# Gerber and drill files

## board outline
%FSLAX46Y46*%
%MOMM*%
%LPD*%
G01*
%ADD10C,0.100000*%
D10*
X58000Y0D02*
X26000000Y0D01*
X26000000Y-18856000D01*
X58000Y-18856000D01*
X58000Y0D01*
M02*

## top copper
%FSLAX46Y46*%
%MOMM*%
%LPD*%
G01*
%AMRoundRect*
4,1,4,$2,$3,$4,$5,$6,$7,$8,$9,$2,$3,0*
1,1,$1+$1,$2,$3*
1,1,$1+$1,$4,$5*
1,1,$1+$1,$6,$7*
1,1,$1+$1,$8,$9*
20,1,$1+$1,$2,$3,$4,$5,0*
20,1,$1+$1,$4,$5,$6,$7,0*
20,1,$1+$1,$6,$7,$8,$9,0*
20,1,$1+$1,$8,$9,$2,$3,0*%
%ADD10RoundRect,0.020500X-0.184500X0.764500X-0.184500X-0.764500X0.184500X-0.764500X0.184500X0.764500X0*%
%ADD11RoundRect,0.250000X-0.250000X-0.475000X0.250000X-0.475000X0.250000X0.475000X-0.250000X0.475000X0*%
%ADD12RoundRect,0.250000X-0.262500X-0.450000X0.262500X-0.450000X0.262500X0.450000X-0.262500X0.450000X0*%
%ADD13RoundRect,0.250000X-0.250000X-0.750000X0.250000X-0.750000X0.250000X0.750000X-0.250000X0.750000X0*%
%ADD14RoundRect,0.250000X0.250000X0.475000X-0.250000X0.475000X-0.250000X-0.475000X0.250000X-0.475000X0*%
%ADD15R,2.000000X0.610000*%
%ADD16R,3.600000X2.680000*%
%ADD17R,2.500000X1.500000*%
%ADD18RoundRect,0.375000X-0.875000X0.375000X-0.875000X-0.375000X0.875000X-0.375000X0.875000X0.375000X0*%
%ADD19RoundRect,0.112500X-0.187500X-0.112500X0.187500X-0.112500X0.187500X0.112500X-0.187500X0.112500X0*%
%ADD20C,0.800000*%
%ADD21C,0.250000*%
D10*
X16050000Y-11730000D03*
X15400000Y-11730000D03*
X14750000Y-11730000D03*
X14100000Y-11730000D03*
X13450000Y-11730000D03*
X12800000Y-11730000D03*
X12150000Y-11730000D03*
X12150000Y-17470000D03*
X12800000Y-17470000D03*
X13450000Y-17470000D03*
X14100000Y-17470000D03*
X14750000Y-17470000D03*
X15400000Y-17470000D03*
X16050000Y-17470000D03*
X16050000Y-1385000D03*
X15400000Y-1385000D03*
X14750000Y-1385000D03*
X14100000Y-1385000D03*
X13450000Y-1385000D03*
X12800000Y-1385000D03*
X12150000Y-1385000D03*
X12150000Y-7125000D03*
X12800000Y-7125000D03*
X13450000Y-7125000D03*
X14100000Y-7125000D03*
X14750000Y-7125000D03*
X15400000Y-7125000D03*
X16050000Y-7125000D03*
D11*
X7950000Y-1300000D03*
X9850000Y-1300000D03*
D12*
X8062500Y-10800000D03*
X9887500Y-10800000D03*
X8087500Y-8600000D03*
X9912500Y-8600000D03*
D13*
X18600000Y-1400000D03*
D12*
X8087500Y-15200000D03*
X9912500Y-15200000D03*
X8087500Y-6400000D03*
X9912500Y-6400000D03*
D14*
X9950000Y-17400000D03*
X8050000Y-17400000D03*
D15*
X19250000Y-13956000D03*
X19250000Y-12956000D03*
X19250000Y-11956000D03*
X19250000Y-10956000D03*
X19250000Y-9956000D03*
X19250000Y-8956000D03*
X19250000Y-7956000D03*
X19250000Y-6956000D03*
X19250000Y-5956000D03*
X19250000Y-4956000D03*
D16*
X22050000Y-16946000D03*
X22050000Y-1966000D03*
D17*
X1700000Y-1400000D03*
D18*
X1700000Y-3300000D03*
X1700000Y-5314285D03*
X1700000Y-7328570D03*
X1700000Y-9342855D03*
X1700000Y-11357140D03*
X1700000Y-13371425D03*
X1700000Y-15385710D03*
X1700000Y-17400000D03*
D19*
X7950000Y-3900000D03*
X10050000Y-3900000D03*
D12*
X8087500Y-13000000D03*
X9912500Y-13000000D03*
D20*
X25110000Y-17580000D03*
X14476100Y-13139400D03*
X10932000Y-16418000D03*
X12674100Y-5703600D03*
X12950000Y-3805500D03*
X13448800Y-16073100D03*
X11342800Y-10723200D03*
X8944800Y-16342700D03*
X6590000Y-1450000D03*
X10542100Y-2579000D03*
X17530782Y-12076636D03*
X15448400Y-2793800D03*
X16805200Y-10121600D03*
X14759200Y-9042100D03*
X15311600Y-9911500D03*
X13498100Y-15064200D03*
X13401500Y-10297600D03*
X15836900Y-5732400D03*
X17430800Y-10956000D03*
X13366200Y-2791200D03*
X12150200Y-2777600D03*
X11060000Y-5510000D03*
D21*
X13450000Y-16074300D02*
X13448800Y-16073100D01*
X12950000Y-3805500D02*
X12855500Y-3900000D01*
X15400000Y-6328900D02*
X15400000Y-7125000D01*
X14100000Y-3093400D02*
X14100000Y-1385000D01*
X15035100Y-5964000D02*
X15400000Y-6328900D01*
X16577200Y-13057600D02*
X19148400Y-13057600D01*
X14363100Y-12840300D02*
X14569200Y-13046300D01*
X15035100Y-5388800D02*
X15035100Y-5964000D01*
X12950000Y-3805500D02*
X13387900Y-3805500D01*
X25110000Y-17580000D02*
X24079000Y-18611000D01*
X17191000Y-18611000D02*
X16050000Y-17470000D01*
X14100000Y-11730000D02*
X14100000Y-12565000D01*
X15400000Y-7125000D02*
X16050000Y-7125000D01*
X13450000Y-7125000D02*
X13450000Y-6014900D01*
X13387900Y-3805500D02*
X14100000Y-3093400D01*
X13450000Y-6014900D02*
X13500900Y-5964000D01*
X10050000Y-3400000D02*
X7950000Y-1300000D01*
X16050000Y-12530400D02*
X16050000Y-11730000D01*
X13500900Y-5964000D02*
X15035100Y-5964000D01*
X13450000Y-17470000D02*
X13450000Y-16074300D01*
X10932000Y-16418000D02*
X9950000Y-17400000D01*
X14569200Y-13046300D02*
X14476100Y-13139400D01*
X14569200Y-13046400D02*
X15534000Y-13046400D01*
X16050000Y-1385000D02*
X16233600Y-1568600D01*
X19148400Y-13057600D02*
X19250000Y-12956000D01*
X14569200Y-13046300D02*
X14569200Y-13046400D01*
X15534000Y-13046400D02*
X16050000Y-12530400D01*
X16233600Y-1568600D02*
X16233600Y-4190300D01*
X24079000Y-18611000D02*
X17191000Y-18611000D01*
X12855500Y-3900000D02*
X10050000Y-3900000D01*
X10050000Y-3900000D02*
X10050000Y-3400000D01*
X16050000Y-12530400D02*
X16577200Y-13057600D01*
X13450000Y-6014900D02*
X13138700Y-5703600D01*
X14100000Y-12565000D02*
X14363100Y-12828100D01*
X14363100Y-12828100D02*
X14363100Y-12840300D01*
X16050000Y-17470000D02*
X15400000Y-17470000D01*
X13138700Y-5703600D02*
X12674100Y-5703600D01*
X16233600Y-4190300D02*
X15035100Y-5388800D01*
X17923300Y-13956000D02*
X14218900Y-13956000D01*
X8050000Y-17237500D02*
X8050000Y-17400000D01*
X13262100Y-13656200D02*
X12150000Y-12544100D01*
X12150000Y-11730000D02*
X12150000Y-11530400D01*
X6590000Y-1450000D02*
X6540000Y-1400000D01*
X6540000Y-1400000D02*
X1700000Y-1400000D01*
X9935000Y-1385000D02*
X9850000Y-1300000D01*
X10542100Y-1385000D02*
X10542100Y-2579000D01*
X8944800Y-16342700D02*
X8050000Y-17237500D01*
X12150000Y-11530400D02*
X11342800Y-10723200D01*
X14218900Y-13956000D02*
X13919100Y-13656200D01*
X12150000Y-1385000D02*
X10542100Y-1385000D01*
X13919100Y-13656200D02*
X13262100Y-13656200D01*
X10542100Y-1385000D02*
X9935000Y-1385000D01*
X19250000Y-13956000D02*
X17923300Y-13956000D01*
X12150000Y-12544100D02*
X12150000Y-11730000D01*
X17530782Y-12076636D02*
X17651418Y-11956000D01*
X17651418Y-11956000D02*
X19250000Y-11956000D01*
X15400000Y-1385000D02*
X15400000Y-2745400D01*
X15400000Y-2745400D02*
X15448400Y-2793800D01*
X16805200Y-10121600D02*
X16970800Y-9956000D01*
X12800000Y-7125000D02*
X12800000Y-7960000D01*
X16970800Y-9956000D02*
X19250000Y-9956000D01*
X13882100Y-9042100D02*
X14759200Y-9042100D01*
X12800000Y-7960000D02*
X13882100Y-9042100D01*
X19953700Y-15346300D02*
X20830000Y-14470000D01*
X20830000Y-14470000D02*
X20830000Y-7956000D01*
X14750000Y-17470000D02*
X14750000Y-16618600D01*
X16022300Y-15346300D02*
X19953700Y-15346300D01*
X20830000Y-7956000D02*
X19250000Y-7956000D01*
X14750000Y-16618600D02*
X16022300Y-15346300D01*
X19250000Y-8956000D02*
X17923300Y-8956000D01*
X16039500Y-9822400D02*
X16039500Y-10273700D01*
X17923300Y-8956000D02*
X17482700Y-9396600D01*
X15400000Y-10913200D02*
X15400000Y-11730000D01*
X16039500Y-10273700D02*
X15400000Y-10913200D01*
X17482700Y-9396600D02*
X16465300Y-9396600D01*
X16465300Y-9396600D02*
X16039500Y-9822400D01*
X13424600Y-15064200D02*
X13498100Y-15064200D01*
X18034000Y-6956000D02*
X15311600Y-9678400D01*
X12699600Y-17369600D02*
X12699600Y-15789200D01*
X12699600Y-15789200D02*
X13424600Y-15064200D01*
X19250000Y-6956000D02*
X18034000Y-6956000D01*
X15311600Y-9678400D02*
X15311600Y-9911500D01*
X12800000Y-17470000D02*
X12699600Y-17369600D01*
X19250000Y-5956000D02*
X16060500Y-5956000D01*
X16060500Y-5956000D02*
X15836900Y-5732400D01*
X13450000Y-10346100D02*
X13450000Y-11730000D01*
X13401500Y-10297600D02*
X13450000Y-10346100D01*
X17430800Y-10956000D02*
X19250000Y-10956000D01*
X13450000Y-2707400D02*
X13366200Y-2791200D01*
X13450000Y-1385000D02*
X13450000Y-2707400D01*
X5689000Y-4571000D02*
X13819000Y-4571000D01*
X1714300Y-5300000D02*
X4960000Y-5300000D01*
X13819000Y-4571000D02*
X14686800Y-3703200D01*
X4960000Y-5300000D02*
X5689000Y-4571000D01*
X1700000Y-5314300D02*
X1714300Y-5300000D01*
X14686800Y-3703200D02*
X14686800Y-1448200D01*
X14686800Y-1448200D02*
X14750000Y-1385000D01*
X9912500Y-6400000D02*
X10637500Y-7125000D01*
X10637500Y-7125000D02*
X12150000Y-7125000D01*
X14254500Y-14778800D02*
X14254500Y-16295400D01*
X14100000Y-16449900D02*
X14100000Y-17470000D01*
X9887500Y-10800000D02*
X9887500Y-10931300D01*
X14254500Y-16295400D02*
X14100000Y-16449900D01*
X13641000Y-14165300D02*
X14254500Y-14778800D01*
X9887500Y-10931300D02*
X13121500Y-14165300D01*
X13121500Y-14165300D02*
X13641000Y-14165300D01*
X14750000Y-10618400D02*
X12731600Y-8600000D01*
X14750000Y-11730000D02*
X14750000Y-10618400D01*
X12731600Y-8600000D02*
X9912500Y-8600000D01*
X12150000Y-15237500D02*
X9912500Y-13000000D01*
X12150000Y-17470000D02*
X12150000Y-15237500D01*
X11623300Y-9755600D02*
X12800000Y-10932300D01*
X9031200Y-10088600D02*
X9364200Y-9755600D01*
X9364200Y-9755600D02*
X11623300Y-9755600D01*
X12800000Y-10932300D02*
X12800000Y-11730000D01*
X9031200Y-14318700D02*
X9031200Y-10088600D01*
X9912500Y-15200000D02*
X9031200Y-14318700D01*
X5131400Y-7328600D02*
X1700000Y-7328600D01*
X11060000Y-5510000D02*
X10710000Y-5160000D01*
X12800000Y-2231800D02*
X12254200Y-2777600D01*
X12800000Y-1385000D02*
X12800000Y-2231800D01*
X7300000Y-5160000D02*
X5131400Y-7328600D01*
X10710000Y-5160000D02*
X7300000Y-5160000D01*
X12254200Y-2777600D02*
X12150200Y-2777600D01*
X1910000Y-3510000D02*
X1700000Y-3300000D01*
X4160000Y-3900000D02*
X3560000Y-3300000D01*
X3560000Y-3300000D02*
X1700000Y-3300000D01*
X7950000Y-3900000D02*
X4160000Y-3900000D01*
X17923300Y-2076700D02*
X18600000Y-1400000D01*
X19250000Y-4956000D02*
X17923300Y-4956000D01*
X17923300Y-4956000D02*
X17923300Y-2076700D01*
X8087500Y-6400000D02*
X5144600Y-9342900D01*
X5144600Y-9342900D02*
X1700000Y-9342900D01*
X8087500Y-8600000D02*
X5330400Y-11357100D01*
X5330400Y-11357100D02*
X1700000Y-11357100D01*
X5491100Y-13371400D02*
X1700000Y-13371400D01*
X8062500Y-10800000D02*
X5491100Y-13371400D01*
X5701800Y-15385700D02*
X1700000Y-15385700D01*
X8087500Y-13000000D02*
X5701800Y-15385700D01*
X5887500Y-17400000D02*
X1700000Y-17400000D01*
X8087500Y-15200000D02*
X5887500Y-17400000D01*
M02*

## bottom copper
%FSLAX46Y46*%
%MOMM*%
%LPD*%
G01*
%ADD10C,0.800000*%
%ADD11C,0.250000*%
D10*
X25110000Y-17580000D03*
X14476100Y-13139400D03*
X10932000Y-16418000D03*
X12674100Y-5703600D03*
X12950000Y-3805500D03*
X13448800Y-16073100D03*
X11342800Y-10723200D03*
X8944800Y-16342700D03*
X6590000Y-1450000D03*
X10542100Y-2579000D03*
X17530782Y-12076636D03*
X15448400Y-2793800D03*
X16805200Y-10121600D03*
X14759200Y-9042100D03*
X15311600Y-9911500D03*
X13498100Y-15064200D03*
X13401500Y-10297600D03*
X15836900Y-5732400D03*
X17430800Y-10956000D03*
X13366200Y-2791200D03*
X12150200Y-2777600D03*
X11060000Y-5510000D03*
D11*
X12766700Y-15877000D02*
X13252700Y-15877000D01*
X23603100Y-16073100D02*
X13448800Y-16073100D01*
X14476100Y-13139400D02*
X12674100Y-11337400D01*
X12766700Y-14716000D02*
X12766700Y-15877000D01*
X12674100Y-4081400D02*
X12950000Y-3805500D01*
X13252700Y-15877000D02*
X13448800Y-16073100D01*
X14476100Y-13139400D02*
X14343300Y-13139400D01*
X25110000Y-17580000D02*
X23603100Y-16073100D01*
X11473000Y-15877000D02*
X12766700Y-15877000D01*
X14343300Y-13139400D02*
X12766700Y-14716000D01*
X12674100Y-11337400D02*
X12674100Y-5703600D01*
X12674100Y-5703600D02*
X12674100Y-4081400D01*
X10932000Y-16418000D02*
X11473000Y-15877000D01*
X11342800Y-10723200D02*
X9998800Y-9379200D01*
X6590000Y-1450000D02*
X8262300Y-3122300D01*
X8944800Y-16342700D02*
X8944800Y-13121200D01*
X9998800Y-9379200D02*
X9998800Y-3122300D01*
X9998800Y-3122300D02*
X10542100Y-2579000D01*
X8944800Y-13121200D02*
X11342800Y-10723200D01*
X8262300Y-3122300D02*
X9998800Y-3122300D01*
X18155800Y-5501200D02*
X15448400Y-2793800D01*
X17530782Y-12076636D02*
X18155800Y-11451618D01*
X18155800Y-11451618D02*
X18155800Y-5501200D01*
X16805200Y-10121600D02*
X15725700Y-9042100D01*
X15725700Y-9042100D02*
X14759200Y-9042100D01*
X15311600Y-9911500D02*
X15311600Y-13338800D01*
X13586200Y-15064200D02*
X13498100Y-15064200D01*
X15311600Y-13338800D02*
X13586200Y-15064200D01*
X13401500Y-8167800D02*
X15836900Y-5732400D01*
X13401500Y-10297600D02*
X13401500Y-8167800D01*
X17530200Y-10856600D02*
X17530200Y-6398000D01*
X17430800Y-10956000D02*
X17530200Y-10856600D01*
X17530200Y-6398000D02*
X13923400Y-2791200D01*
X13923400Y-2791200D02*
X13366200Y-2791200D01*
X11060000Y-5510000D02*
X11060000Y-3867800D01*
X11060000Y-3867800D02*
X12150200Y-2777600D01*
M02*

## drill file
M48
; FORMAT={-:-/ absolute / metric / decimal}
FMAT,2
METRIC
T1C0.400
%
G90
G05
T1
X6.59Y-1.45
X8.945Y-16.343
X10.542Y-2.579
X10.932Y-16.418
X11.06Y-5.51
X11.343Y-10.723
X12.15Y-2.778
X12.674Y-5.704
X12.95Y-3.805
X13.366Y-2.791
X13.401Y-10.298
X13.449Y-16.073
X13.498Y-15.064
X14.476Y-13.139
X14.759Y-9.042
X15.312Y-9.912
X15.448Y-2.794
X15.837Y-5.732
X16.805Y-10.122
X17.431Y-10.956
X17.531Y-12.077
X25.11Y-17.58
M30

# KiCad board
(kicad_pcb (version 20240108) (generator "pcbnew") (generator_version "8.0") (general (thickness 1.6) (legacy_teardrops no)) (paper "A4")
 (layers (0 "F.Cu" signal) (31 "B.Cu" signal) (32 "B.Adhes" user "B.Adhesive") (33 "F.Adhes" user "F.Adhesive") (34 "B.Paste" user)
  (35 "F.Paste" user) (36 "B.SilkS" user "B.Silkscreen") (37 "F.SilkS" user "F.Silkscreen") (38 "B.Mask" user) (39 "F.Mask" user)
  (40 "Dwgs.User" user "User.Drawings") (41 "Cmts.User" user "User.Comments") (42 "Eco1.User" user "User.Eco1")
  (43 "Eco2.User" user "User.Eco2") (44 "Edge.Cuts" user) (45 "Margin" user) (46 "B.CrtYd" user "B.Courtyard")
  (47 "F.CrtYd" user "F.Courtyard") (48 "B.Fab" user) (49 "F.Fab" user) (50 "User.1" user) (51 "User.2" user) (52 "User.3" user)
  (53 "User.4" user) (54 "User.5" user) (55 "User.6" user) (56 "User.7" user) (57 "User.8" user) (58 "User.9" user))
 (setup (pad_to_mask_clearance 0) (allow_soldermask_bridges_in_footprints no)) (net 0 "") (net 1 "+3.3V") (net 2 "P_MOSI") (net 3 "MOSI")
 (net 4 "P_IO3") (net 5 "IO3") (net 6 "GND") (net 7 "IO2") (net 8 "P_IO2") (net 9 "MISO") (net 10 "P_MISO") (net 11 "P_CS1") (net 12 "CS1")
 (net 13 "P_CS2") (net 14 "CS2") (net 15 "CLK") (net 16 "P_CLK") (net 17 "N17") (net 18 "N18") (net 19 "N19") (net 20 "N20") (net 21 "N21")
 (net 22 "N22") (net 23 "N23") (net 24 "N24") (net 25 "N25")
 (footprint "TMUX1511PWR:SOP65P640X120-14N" (layer "F.Cu") (at 14.1 14.6 -90)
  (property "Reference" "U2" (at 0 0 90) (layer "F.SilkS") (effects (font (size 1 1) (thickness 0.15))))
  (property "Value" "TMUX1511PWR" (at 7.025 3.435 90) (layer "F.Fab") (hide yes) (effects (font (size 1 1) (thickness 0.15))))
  (pad "1" smd roundrect (at -2.87 -1.95 270) (size 1.57 0.41) (layers "F.Cu" "F.Paste" "F.Mask") (roundrect_rratio 0.05) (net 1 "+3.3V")
   (solder_mask_margin 0.102))
  (pad "2" smd roundrect (at -2.87 -1.3 270) (size 1.57 0.41) (layers "F.Cu" "F.Paste" "F.Mask") (roundrect_rratio 0.05) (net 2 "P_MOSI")
   (solder_mask_margin 0.102))
  (pad "3" smd roundrect (at -2.87 -0.65 270) (size 1.57 0.41) (layers "F.Cu" "F.Paste" "F.Mask") (roundrect_rratio 0.05) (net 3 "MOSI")
   (solder_mask_margin 0.102))
  (pad "4" smd roundrect (at -2.87 0 270) (size 1.57 0.41) (layers "F.Cu" "F.Paste" "F.Mask") (roundrect_rratio 0.05) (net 1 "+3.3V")
   (solder_mask_margin 0.102))
  (pad "5" smd roundrect (at -2.87 0.65 270) (size 1.57 0.41) (layers "F.Cu" "F.Paste" "F.Mask") (roundrect_rratio 0.05) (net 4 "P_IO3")
   (solder_mask_margin 0.102))
  (pad "6" smd roundrect (at -2.87 1.3 270) (size 1.57 0.41) (layers "F.Cu" "F.Paste" "F.Mask") (roundrect_rratio 0.05) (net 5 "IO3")
   (solder_mask_margin 0.102))
  (pad "7" smd roundrect (at -2.87 1.95 270) (size 1.57 0.41) (layers "F.Cu" "F.Paste" "F.Mask") (roundrect_rratio 0.05) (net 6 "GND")
   (solder_mask_margin 0.102))
  (pad "8" smd roundrect (at 2.87 1.95 270) (size 1.57 0.41) (layers "F.Cu" "F.Paste" "F.Mask") (roundrect_rratio 0.05) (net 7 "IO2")
   (solder_mask_margin 0.102))
  (pad "9" smd roundrect (at 2.87 1.3 270) (size 1.57 0.41) (layers "F.Cu" "F.Paste" "F.Mask") (roundrect_rratio 0.05) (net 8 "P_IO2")
   (solder_mask_margin 0.102))
  (pad "10" smd roundrect (at 2.87 0.65 270) (size 1.57 0.41) (layers "F.Cu" "F.Paste" "F.Mask") (roundrect_rratio 0.05) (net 1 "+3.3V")
   (solder_mask_margin 0.102))
  (pad "11" smd roundrect (at 2.87 0 270) (size 1.57 0.41) (layers "F.Cu" "F.Paste" "F.Mask") (roundrect_rratio 0.05) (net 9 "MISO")
   (solder_mask_margin 0.102))
  (pad "12" smd roundrect (at 2.87 -0.65 270) (size 1.57 0.41) (layers "F.Cu" "F.Paste" "F.Mask") (roundrect_rratio 0.05) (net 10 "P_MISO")
   (solder_mask_margin 0.102))
  (pad "13" smd roundrect (at 2.87 -1.3 270) (size 1.57 0.41) (layers "F.Cu" "F.Paste" "F.Mask") (roundrect_rratio 0.05) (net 1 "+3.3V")
   (solder_mask_margin 0.102))
  (pad "14" smd roundrect (at 2.87 -1.95 270) (size 1.57 0.41) (layers "F.Cu" "F.Paste" "F.Mask") (roundrect_rratio 0.05) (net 1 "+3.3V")
   (solder_mask_margin 0.102)))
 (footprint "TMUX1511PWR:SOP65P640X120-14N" (layer "F.Cu") (at 14.1 4.255 -90)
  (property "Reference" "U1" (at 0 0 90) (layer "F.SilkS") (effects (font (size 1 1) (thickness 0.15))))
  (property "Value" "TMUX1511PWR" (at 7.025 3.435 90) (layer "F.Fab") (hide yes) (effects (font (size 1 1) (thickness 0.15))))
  (pad "1" smd roundrect (at -2.87 -1.95 270) (size 1.57 0.41) (layers "F.Cu" "F.Paste" "F.Mask") (roundrect_rratio 0.05) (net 1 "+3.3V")
   (solder_mask_margin 0.102))
  (pad "2" smd roundrect (at -2.87 -1.3 270) (size 1.57 0.41) (layers "F.Cu" "F.Paste" "F.Mask") (roundrect_rratio 0.05) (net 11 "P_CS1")
   (solder_mask_margin 0.102))
  (pad "3" smd roundrect (at -2.87 -0.65 270) (size 1.57 0.41) (layers "F.Cu" "F.Paste" "F.Mask") (roundrect_rratio 0.05) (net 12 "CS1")
   (solder_mask_margin 0.102))
  (pad "4" smd roundrect (at -2.87 0 270) (size 1.57 0.41) (layers "F.Cu" "F.Paste" "F.Mask") (roundrect_rratio 0.05) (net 1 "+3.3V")
   (solder_mask_margin 0.102))
  (pad "5" smd roundrect (at -2.87 0.65 270) (size 1.57 0.41) (layers "F.Cu" "F.Paste" "F.Mask") (roundrect_rratio 0.05) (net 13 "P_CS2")
   (solder_mask_margin 0.102))
  (pad "6" smd roundrect (at -2.87 1.3 270) (size 1.57 0.41) (layers "F.Cu" "F.Paste" "F.Mask") (roundrect_rratio 0.05) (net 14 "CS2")
   (solder_mask_margin 0.102))
  (pad "7" smd roundrect (at -2.87 1.95 270) (size 1.57 0.41) (layers "F.Cu" "F.Paste" "F.Mask") (roundrect_rratio 0.05) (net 6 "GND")
   (solder_mask_margin 0.102))
  (pad "8" smd roundrect (at 2.87 1.95 270) (size 1.57 0.41) (layers "F.Cu" "F.Paste" "F.Mask") (roundrect_rratio 0.05) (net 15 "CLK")
   (solder_mask_margin 0.102))
  (pad "9" smd roundrect (at 2.87 1.3 270) (size 1.57 0.41) (layers "F.Cu" "F.Paste" "F.Mask") (roundrect_rratio 0.05) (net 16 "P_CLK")
   (solder_mask_margin 0.102))
  (pad "10" smd roundrect (at 2.87 0.65 270) (size 1.57 0.41) (layers "F.Cu" "F.Paste" "F.Mask") (roundrect_rratio 0.05) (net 1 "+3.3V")
   (solder_mask_margin 0.102))
  (pad "11" smd roundrect (at 2.87 0 270) (size 1.57 0.41) (layers "F.Cu" "F.Paste" "F.Mask") (roundrect_rratio 0.05) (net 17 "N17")
   (solder_mask_margin 0.102))
  (pad "12" smd roundrect (at 2.87 -0.65 270) (size 1.57 0.41) (layers "F.Cu" "F.Paste" "F.Mask") (roundrect_rratio 0.05) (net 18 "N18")
   (solder_mask_margin 0.102))
  (pad "13" smd roundrect (at 2.87 -1.3 270) (size 1.57 0.41) (layers "F.Cu" "F.Paste" "F.Mask") (roundrect_rratio 0.05) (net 1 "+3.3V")
   (solder_mask_margin 0.102))
  (pad "14" smd roundrect (at 2.87 -1.95 270) (size 1.57 0.41) (layers "F.Cu" "F.Paste" "F.Mask") (roundrect_rratio 0.05) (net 1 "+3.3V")
   (solder_mask_margin 0.102)))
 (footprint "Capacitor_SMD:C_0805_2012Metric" (layer "F.Cu") (at 8.9 1.3)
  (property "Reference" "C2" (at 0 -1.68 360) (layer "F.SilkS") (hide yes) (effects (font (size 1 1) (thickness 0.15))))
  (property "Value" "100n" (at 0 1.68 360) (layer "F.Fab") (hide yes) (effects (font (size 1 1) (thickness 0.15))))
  (pad "1" smd roundrect (at -0.95 0) (size 1 1.45) (layers "F.Cu" "F.Paste" "F.Mask") (roundrect_rratio 0.25) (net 1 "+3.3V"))
  (pad "2" smd roundrect (at 0.95 0) (size 1 1.45) (layers "F.Cu" "F.Paste" "F.Mask") (roundrect_rratio 0.25) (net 6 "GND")))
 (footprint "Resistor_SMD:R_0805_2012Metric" (layer "F.Cu") (at 8.975 10.8)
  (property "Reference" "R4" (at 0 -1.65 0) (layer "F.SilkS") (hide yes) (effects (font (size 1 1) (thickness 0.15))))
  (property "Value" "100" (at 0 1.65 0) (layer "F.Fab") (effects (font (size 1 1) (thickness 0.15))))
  (pad "1" smd roundrect (at -0.9125 0) (size 1.025 1.4) (layers "F.Cu" "F.Paste" "F.Mask") (roundrect_rratio 0.243902439) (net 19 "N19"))
  (pad "2" smd roundrect (at 0.9125 0) (size 1.025 1.4) (layers "F.Cu" "F.Paste" "F.Mask") (roundrect_rratio 0.243902439) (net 9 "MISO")))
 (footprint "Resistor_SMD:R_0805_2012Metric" (layer "F.Cu") (at 9 8.6)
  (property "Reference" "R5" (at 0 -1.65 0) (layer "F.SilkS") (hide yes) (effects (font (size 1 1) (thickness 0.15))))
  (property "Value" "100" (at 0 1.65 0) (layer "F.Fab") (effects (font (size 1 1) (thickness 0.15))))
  (pad "1" smd roundrect (at -0.9125 0) (size 1.025 1.4) (layers "F.Cu" "F.Paste" "F.Mask") (roundrect_rratio 0.243902439) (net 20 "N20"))
  (pad "2" smd roundrect (at 0.9125 0) (size 1.025 1.4) (layers "F.Cu" "F.Paste" "F.Mask") (roundrect_rratio 0.243902439) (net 3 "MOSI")))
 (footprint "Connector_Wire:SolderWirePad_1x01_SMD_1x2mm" (layer "F.Cu") (at 18.6 1.4)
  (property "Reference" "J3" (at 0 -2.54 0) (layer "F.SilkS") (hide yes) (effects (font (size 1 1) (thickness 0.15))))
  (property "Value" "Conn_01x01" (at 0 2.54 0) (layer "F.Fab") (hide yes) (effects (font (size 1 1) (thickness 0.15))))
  (pad "1" smd roundrect (at 0 0) (size 1 2) (layers "F.Cu" "F.Paste" "F.Mask") (roundrect_rratio 0.25) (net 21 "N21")))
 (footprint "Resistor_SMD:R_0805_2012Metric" (layer "F.Cu") (at 9 15.2)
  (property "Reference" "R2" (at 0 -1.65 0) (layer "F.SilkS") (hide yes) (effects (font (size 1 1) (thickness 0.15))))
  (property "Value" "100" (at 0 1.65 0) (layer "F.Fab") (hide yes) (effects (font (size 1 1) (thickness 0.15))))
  (pad "1" smd roundrect (at -0.9125 0) (size 1.025 1.4) (layers "F.Cu" "F.Paste" "F.Mask") (roundrect_rratio 0.243902439) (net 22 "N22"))
  (pad "2" smd roundrect (at 0.9125 0) (size 1.025 1.4) (layers "F.Cu" "F.Paste" "F.Mask") (roundrect_rratio 0.243902439) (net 5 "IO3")))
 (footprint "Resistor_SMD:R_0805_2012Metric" (layer "F.Cu") (at 9 6.4)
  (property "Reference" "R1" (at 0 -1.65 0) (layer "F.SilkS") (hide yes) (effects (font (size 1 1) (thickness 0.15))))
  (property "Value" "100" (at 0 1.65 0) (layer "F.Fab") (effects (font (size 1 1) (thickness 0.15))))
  (pad "1" smd roundrect (at -0.9125 0) (size 1.025 1.4) (layers "F.Cu" "F.Paste" "F.Mask") (roundrect_rratio 0.243902439) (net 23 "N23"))
  (pad "2" smd roundrect (at 0.9125 0) (size 1.025 1.4) (layers "F.Cu" "F.Paste" "F.Mask") (roundrect_rratio 0.243902439) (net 15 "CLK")))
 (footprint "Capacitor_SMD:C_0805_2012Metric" (layer "F.Cu") (at 9 17.4 180)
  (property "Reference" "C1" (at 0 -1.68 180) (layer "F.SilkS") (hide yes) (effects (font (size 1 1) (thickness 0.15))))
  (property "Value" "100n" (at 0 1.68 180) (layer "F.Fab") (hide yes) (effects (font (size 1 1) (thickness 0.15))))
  (pad "1" smd roundrect (at -0.95 0 180) (size 1 1.45) (layers "F.Cu" "F.Paste" "F.Mask") (roundrect_rratio 0.25) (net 1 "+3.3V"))
  (pad "2" smd roundrect (at 0.95 0 180) (size 1 1.45) (layers "F.Cu" "F.Paste" "F.Mask") (roundrect_rratio 0.25) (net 6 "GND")))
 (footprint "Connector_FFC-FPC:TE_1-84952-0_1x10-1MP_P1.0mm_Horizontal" (layer "F.Cu") (at 21.05 9.456 90)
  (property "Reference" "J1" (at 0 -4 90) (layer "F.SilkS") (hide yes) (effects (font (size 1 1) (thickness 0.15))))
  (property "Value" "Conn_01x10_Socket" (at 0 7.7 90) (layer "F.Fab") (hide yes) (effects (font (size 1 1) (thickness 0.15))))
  (pad "1" smd rect (at -4.5 -1.8 90) (size 0.61 2) (layers "F.Cu" "F.Paste" "F.Mask") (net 6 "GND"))
  (pad "2" smd rect (at -3.5 -1.8 90) (size 0.61 2) (layers "F.Cu" "F.Paste" "F.Mask") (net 1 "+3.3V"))
  (pad "3" smd rect (at -2.5 -1.8 90) (size 0.61 2) (layers "F.Cu" "F.Paste" "F.Mask") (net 11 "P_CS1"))
  (pad "4" smd rect (at -1.5 -1.8 90) (size 0.61 2) (layers "F.Cu" "F.Paste" "F.Mask") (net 13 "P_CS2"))
  (pad "5" smd rect (at -0.5 -1.8 90) (size 0.61 2) (layers "F.Cu" "F.Paste" "F.Mask") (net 16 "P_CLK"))
  (pad "6" smd rect (at 0.5 -1.8 90) (size 0.61 2) (layers "F.Cu" "F.Paste" "F.Mask") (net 2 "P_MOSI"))
  (pad "7" smd rect (at 1.5 -1.8 90) (size 0.61 2) (layers "F.Cu" "F.Paste" "F.Mask") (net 10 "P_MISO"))
  (pad "8" smd rect (at 2.5 -1.8 90) (size 0.61 2) (layers "F.Cu" "F.Paste" "F.Mask") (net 8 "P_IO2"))
  (pad "9" smd rect (at 3.5 -1.8 90) (size 0.61 2) (layers "F.Cu" "F.Paste" "F.Mask") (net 4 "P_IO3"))
  (pad "10" smd rect (at 4.5 -1.8 90) (size 0.61 2) (layers "F.Cu" "F.Paste" "F.Mask") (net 21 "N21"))
  (pad "MP" smd rect (at -7.49 1 90) (size 2.68 3.6) (layers "F.Cu" "F.Paste" "F.Mask"))
  (pad "MP" smd rect (at 7.49 1 90) (size 2.68 3.6) (layers "F.Cu" "F.Paste" "F.Mask")))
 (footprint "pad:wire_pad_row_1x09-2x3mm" (layer "F.Cu") (at 1.7 1.4 -90)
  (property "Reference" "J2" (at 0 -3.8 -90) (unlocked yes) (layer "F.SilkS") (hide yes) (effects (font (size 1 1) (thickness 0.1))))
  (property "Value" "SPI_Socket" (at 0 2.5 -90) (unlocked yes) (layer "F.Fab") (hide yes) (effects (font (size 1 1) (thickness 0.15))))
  (pad "1" smd rect (at 0 0 270) (size 1.5 2.5) (layers "F.Cu" "F.Paste" "F.Mask") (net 6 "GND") (thermal_bridge_angle 45))
  (pad "2" smd roundrect (at 1.9 0 270) (size 1.5 2.5) (layers "F.Cu" "F.Paste" "F.Mask") (roundrect_rratio 0.25) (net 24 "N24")
   (thermal_bridge_angle 45))
  (pad "3" smd roundrect (at 3.914285 0 270) (size 1.5 2.5) (layers "F.Cu" "F.Paste" "F.Mask") (roundrect_rratio 0.25) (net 12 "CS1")
   (thermal_bridge_angle 45))
  (pad "4" smd roundrect (at 5.92857 0 270) (size 1.5 2.5) (layers "F.Cu" "F.Paste" "F.Mask") (roundrect_rratio 0.25) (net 14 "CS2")
   (thermal_bridge_angle 45))
  (pad "5" smd roundrect (at 7.942855 0 270) (size 1.5 2.5) (layers "F.Cu" "F.Paste" "F.Mask") (roundrect_rratio 0.25) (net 23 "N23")
   (thermal_bridge_angle 45))
  (pad "6" smd roundrect (at 9.95714 0 270) (size 1.5 2.5) (layers "F.Cu" "F.Paste" "F.Mask") (roundrect_rratio 0.25) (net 20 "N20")
   (thermal_bridge_angle 45))
  (pad "7" smd roundrect (at 11.971425 0 270) (size 1.5 2.5) (layers "F.Cu" "F.Paste" "F.Mask") (roundrect_rratio 0.25) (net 19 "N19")
   (thermal_bridge_angle 45))
  (pad "8" smd roundrect (at 13.98571 0 270) (size 1.5 2.5) (layers "F.Cu" "F.Paste" "F.Mask") (roundrect_rratio 0.25) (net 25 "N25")
   (thermal_bridge_angle 45))
  (pad "9" smd roundrect (at 16 0 270) (size 1.5 2.5) (layers "F.Cu" "F.Paste" "F.Mask") (roundrect_rratio 0.25) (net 22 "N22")
   (thermal_bridge_angle 45)))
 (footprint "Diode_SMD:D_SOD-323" (layer "F.Cu") (at 9 3.9)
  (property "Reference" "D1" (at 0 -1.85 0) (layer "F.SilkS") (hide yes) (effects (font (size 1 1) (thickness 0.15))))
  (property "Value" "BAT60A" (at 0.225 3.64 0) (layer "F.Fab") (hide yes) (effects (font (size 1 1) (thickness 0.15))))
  (pad "1" smd roundrect (at -1.05 0) (size 0.6 0.45) (layers "F.Cu" "F.Paste" "F.Mask") (roundrect_rratio 0.25) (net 24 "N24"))
  (pad "2" smd roundrect (at 1.05 0) (size 0.6 0.45) (layers "F.Cu" "F.Paste" "F.Mask") (roundrect_rratio 0.25) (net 1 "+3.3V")))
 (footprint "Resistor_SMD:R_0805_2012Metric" (layer "F.Cu") (at 9 13)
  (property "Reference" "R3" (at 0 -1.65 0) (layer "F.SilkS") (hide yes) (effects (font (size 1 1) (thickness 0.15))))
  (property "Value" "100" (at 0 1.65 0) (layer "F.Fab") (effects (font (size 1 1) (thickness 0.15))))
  (pad "1" smd roundrect (at -0.9125 0) (size 1.025 1.4) (layers "F.Cu" "F.Paste" "F.Mask") (roundrect_rratio 0.243902439) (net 25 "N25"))
  (pad "2" smd roundrect (at 0.9125 0) (size 1.025 1.4) (layers "F.Cu" "F.Paste" "F.Mask") (roundrect_rratio 0.243902439) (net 7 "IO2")))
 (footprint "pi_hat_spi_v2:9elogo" (layer "B.Cu") (at 21 14.9 180)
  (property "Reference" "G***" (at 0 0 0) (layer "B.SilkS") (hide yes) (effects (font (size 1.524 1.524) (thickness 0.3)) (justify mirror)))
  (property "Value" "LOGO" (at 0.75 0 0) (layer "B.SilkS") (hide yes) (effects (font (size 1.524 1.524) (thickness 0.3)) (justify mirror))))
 (gr_rect (start 0.058 0) (end 26 18.856) (stroke (width 0.1) (type default)) (fill none) (layer "Edge.Cuts"))
 (segment (start 13.45 16.0743) (end 13.4488 16.0731) (width 0.25) (layer "F.Cu") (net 1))
 (segment (start 12.95 3.8055) (end 12.8555 3.9) (width 0.25) (layer "F.Cu") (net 1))
 (segment (start 15.4 6.3289) (end 15.4 7.125) (width 0.25) (layer "F.Cu") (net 1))
 (segment (start 14.1 3.0934) (end 14.1 1.385) (width 0.25) (layer "F.Cu") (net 1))
 (segment (start 15.0351 5.964) (end 15.4 6.3289) (width 0.25) (layer "F.Cu") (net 1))
 (segment (start 16.5772 13.0576) (end 19.1484 13.0576) (width 0.25) (layer "F.Cu") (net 1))
 (segment (start 14.3631 12.8403) (end 14.5692 13.0463) (width 0.25) (layer "F.Cu") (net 1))
 (segment (start 15.0351 5.3888) (end 15.0351 5.964) (width 0.25) (layer "F.Cu") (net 1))
 (segment (start 12.95 3.8055) (end 13.3879 3.8055) (width 0.25) (layer "F.Cu") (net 1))
 (segment (start 25.11 17.58) (end 24.079 18.611) (width 0.25) (layer "F.Cu") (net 1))
 (segment (start 17.191 18.611) (end 16.05 17.47) (width 0.25) (layer "F.Cu") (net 1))
 (segment (start 14.1 11.73) (end 14.1 12.565) (width 0.25) (layer "F.Cu") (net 1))
 (segment (start 15.4 7.125) (end 16.05 7.125) (width 0.25) (layer "F.Cu") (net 1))
 (segment (start 13.45 7.125) (end 13.45 6.0149) (width 0.25) (layer "F.Cu") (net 1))
 (segment (start 13.3879 3.8055) (end 14.1 3.0934) (width 0.25) (layer "F.Cu") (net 1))
 (segment (start 13.45 6.0149) (end 13.5009 5.964) (width 0.25) (layer "F.Cu") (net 1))
 (segment (start 10.05 3.4) (end 7.95 1.3) (width 0.25) (layer "F.Cu") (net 1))
 (segment (start 16.05 12.5304) (end 16.05 11.73) (width 0.25) (layer "F.Cu") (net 1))
 (segment (start 13.5009 5.964) (end 15.0351 5.964) (width 0.25) (layer "F.Cu") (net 1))
 (segment (start 13.45 17.47) (end 13.45 16.0743) (width 0.25) (layer "F.Cu") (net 1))
 (segment (start 10.932 16.418) (end 9.95 17.4) (width 0.25) (layer "F.Cu") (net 1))
 (segment (start 14.5692 13.0463) (end 14.4761 13.1394) (width 0.25) (layer "F.Cu") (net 1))
 (segment (start 14.5692 13.0464) (end 15.534 13.0464) (width 0.25) (layer "F.Cu") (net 1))
 (segment (start 16.05 1.385) (end 16.2336 1.5686) (width 0.25) (layer "F.Cu") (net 1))
 (segment (start 19.1484 13.0576) (end 19.25 12.956) (width 0.25) (layer "F.Cu") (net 1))
 (segment (start 14.5692 13.0463) (end 14.5692 13.0464) (width 0.25) (layer "F.Cu") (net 1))
 (segment (start 15.534 13.0464) (end 16.05 12.5304) (width 0.25) (layer "F.Cu") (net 1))
 (segment (start 16.2336 1.5686) (end 16.2336 4.1903) (width 0.25) (layer "F.Cu") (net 1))
 (segment (start 24.079 18.611) (end 17.191 18.611) (width 0.25) (layer "F.Cu") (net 1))
 (segment (start 12.8555 3.9) (end 10.05 3.9) (width 0.25) (layer "F.Cu") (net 1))
 (segment (start 10.05 3.9) (end 10.05 3.4) (width 0.25) (layer "F.Cu") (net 1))
 (segment (start 16.05 12.5304) (end 16.5772 13.0576) (width 0.25) (layer "F.Cu") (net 1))
 (segment (start 13.45 6.0149) (end 13.1387 5.7036) (width 0.25) (layer "F.Cu") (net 1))
 (segment (start 14.1 12.565) (end 14.3631 12.8281) (width 0.25) (layer "F.Cu") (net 1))
 (segment (start 14.3631 12.8281) (end 14.3631 12.8403) (width 0.25) (layer "F.Cu") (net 1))
 (segment (start 16.05 17.47) (end 15.4 17.47) (width 0.25) (layer "F.Cu") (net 1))
 (segment (start 13.1387 5.7036) (end 12.6741 5.7036) (width 0.25) (layer "F.Cu") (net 1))
 (segment (start 16.2336 4.1903) (end 15.0351 5.3888) (width 0.25) (layer "F.Cu") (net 1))
 (via (at 25.11 17.58) (size 0.8) (drill 0.4) (layers "F.Cu" "B.Cu") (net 1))
 (via (at 14.4761 13.1394) (size 0.8) (drill 0.4) (layers "F.Cu" "B.Cu") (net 1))
 (via (at 10.932 16.418) (size 0.8) (drill 0.4) (layers "F.Cu" "B.Cu") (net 1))
 (via (at 12.6741 5.7036) (size 0.8) (drill 0.4) (layers "F.Cu" "B.Cu") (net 1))
 (via (at 12.95 3.8055) (size 0.8) (drill 0.4) (layers "F.Cu" "B.Cu") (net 1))
 (via (at 13.4488 16.0731) (size 0.8) (drill 0.4) (layers "F.Cu" "B.Cu") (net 1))
 (segment (start 12.7667 15.877) (end 13.2527 15.877) (width 0.25) (layer "B.Cu") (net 1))
 (segment (start 23.6031 16.0731) (end 13.4488 16.0731) (width 0.25) (layer "B.Cu") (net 1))
 (segment (start 14.4761 13.1394) (end 12.6741 11.3374) (width 0.25) (layer "B.Cu") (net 1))
 (segment (start 12.7667 14.716) (end 12.7667 15.877) (width 0.25) (layer "B.Cu") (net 1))
 (segment (start 12.6741 4.0814) (end 12.95 3.8055) (width 0.25) (layer "B.Cu") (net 1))
 (segment (start 13.2527 15.877) (end 13.4488 16.0731) (width 0.25) (layer "B.Cu") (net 1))
 (segment (start 14.4761 13.1394) (end 14.3433 13.1394) (width 0.25) (layer "B.Cu") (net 1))
 (segment (start 25.11 17.58) (end 23.6031 16.0731) (width 0.25) (layer "B.Cu") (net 1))
 (segment (start 11.473 15.877) (end 12.7667 15.877) (width 0.25) (layer "B.Cu") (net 1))
 (segment (start 14.3433 13.1394) (end 12.7667 14.716) (width 0.25) (layer "B.Cu") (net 1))
 (segment (start 12.6741 11.3374) (end 12.6741 5.7036) (width 0.25) (layer "B.Cu") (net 1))
 (segment (start 12.6741 5.7036) (end 12.6741 4.0814) (width 0.25) (layer "B.Cu") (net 1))
 (segment (start 10.932 16.418) (end 11.473 15.877) (width 0.25) (layer "B.Cu") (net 1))
 (segment (start 17.9233 13.956) (end 14.2189 13.956) (width 0.25) (layer "F.Cu") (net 6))
 (segment (start 8.05 17.2375) (end 8.05 17.4) (width 0.25) (layer "F.Cu") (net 6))
 (segment (start 13.2621 13.6562) (end 12.15 12.5441) (width 0.25) (layer "F.Cu") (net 6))
 (segment (start 12.15 11.73) (end 12.15 11.5304) (width 0.25) (layer "F.Cu") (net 6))
 (segment (start 6.59 1.45) (end 6.54 1.4) (width 0.25) (layer "F.Cu") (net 6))
 (segment (start 6.54 1.4) (end 1.7 1.4) (width 0.25) (layer "F.Cu") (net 6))
 (segment (start 9.935 1.385) (end 9.85 1.3) (width 0.25) (layer "F.Cu") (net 6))
 (segment (start 10.5421 1.385) (end 10.5421 2.579) (width 0.25) (layer "F.Cu") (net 6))
 (segment (start 8.9448 16.3427) (end 8.05 17.2375) (width 0.25) (layer "F.Cu") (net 6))
 (segment (start 12.15 11.5304) (end 11.3428 10.7232) (width 0.25) (layer "F.Cu") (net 6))
 (segment (start 14.2189 13.956) (end 13.9191 13.6562) (width 0.25) (layer "F.Cu") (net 6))
 (segment (start 12.15 1.385) (end 10.5421 1.385) (width 0.25) (layer "F.Cu") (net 6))
 (segment (start 13.9191 13.6562) (end 13.2621 13.6562) (width 0.25) (layer "F.Cu") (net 6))
 (segment (start 10.5421 1.385) (end 9.935 1.385) (width 0.25) (layer "F.Cu") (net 6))
 (segment (start 19.25 13.956) (end 17.9233 13.956) (width 0.25) (layer "F.Cu") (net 6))
 (segment (start 12.15 12.5441) (end 12.15 11.73) (width 0.25) (layer "F.Cu") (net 6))
 (via (at 11.3428 10.7232) (size 0.8) (drill 0.4) (layers "F.Cu" "B.Cu") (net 6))
 (via (at 8.9448 16.3427) (size 0.8) (drill 0.4) (layers "F.Cu" "B.Cu") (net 6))
 (via (at 6.59 1.45) (size 0.8) (drill 0.4) (layers "F.Cu" "B.Cu") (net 6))
 (via (at 10.5421 2.579) (size 0.8) (drill 0.4) (layers "F.Cu" "B.Cu") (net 6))
 (segment (start 11.3428 10.7232) (end 9.9988 9.3792) (width 0.25) (layer "B.Cu") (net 6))
 (segment (start 6.59 1.45) (end 8.2623 3.1223) (width 0.25) (layer "B.Cu") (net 6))
 (segment (start 8.9448 16.3427) (end 8.9448 13.1212) (width 0.25) (layer "B.Cu") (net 6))
 (segment (start 9.9988 9.3792) (end 9.9988 3.1223) (width 0.25) (layer "B.Cu") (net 6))
 (segment (start 9.9988 3.1223) (end 10.5421 2.579) (width 0.25) (layer "B.Cu") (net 6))
 (segment (start 8.9448 13.1212) (end 11.3428 10.7232) (width 0.25) (layer "B.Cu") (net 6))
 (segment (start 8.2623 3.1223) (end 9.9988 3.1223) (width 0.25) (layer "B.Cu") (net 6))
 (segment (start 17.530782 12.076636) (end 17.651418 11.956) (width 0.25) (layer "F.Cu") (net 11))
 (segment (start 17.651418 11.956) (end 19.25 11.956) (width 0.25) (layer "F.Cu") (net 11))
 (segment (start 15.4 1.385) (end 15.4 2.7454) (width 0.25) (layer "F.Cu") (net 11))
 (segment (start 15.4 2.7454) (end 15.4484 2.7938) (width 0.25) (layer "F.Cu") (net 11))
 (via (at 17.530782 12.076636) (size 0.8) (drill 0.4) (layers "F.Cu" "B.Cu") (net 11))
 (via (at 15.4484 2.7938) (size 0.8) (drill 0.4) (layers "F.Cu" "B.Cu") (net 11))
 (segment (start 18.1558 5.5012) (end 15.4484 2.7938) (width 0.25) (layer "B.Cu") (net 11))
 (segment (start 17.530782 12.076636) (end 18.1558 11.451618) (width 0.25) (layer "B.Cu") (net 11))
 (segment (start 18.1558 11.451618) (end 18.1558 5.5012) (width 0.25) (layer "B.Cu") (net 11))
 (segment (start 16.8052 10.1216) (end 16.9708 9.956) (width 0.25) (layer "F.Cu") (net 16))
 (segment (start 12.8 7.125) (end 12.8 7.96) (width 0.25) (layer "F.Cu") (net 16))
 (segment (start 16.9708 9.956) (end 19.25 9.956) (width 0.25) (layer "F.Cu") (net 16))
 (segment (start 13.8821 9.0421) (end 14.7592 9.0421) (width 0.25) (layer "F.Cu") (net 16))
 (segment (start 12.8 7.96) (end 13.8821 9.0421) (width 0.25) (layer "F.Cu") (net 16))
 (via (at 16.8052 10.1216) (size 0.8) (drill 0.4) (layers "F.Cu" "B.Cu") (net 16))
 (via (at 14.7592 9.0421) (size 0.8) (drill 0.4) (layers "F.Cu" "B.Cu") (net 16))
 (segment (start 16.8052 10.1216) (end 15.7257 9.0421) (width 0.25) (layer "B.Cu") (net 16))
 (segment (start 15.7257 9.0421) (end 14.7592 9.0421) (width 0.25) (layer "B.Cu") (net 16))
 (segment (start 19.9537 15.3463) (end 20.83 14.47) (width 0.25) (layer "F.Cu") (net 10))
 (segment (start 20.83 14.47) (end 20.83 7.956) (width 0.25) (layer "F.Cu") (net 10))
 (segment (start 14.75 17.47) (end 14.75 16.6186) (width 0.25) (layer "F.Cu") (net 10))
 (segment (start 16.0223 15.3463) (end 19.9537 15.3463) (width 0.25) (layer "F.Cu") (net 10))
 (segment (start 20.83 7.956) (end 19.25 7.956) (width 0.25) (layer "F.Cu") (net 10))
 (segment (start 14.75 16.6186) (end 16.0223 15.3463) (width 0.25) (layer "F.Cu") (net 10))
 (segment (start 19.25 8.956) (end 17.9233 8.956) (width 0.25) (layer "F.Cu") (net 2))
 (segment (start 16.0395 9.8224) (end 16.0395 10.2737) (width 0.25) (layer "F.Cu") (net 2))
 (segment (start 17.9233 8.956) (end 17.4827 9.3966) (width 0.25) (layer "F.Cu") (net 2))
 (segment (start 15.4 10.9132) (end 15.4 11.73) (width 0.25) (layer "F.Cu") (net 2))
 (segment (start 16.0395 10.2737) (end 15.4 10.9132) (width 0.25) (layer "F.Cu") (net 2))
 (segment (start 17.4827 9.3966) (end 16.4653 9.3966) (width 0.25) (layer "F.Cu") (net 2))
 (segment (start 16.4653 9.3966) (end 16.0395 9.8224) (width 0.25) (layer "F.Cu") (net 2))
 (segment (start 13.4246 15.0642) (end 13.4981 15.0642) (width 0.25) (layer "F.Cu") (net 8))
 (segment (start 18.034 6.956) (end 15.3116 9.6784) (width 0.25) (layer "F.Cu") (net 8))
 (segment (start 12.6996 17.3696) (end 12.6996 15.7892) (width 0.25) (layer "F.Cu") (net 8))
 (segment (start 12.6996 15.7892) (end 13.4246 15.0642) (width 0.25) (layer "F.Cu") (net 8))
 (segment (start 19.25 6.956) (end 18.034 6.956) (width 0.25) (layer "F.Cu") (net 8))
 (segment (start 15.3116 9.6784) (end 15.3116 9.9115) (width 0.25) (layer "F.Cu") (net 8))
 (segment (start 12.8 17.47) (end 12.6996 17.3696) (width 0.25) (layer "F.Cu") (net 8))
 (via (at 15.3116 9.9115) (size 0.8) (drill 0.4) (layers "F.Cu" "B.Cu") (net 8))
 (via (at 13.4981 15.0642) (size 0.8) (drill 0.4) (layers "F.Cu" "B.Cu") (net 8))
 (segment (start 15.3116 9.9115) (end 15.3116 13.3388) (width 0.25) (layer "B.Cu") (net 8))
 (segment (start 13.5862 15.0642) (end 13.4981 15.0642) (width 0.25) (layer "B.Cu") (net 8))
 (segment (start 15.3116 13.3388) (end 13.5862 15.0642) (width 0.25) (layer "B.Cu") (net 8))
 (segment (start 19.25 5.956) (end 16.0605 5.956) (width 0.25) (layer "F.Cu") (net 4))
 (segment (start 16.0605 5.956) (end 15.8369 5.7324) (width 0.25) (layer "F.Cu") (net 4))
 (segment (start 13.45 10.3461) (end 13.45 11.73) (width 0.25) (layer "F.Cu") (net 4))
 (segment (start 13.4015 10.2976) (end 13.45 10.3461) (width 0.25) (layer "F.Cu") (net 4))
 (via (at 13.4015 10.2976) (size 0.8) (drill 0.4) (layers "F.Cu" "B.Cu") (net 4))
 (via (at 15.8369 5.7324) (size 0.8) (drill 0.4) (layers "F.Cu" "B.Cu") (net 4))
 (segment (start 13.4015 8.1678) (end 15.8369 5.7324) (width 0.25) (layer "B.Cu") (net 4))
 (segment (start 13.4015 10.2976) (end 13.4015 8.1678) (width 0.25) (layer "B.Cu") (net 4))
 (segment (start 17.4308 10.956) (end 19.25 10.956) (width 0.25) (layer "F.Cu") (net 13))
 (segment (start 13.45 2.7074) (end 13.3662 2.7912) (width 0.25) (layer "F.Cu") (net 13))
 (segment (start 13.45 1.385) (end 13.45 2.7074) (width 0.25) (layer "F.Cu") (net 13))
 (via (at 17.4308 10.956) (size 0.8) (drill 0.4) (layers "F.Cu" "B.Cu") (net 13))
 (via (at 13.3662 2.7912) (size 0.8) (drill 0.4) (layers "F.Cu" "B.Cu") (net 13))
 (segment (start 17.5302 10.8566) (end 17.5302 6.398) (width 0.25) (layer "B.Cu") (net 13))
 (segment (start 17.4308 10.956) (end 17.5302 10.8566) (width 0.25) (layer "B.Cu") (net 13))
 (segment (start 17.5302 6.398) (end 13.9234 2.7912) (width 0.25) (layer "B.Cu") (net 13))
 (segment (start 13.9234 2.7912) (end 13.3662 2.7912) (width 0.25) (layer "B.Cu") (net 13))
 (segment (start 5.689 4.571) (end 13.819 4.571) (width 0.25) (layer "F.Cu") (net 12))
 (segment (start 1.7143 5.3) (end 4.96 5.3) (width 0.25) (layer "F.Cu") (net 12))
 (segment (start 13.819 4.571) (end 14.6868 3.7032) (width 0.25) (layer "F.Cu") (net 12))
 (segment (start 4.96 5.3) (end 5.689 4.571) (width 0.25) (layer "F.Cu") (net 12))
 (segment (start 1.7 5.3143) (end 1.7143 5.3) (width 0.25) (layer "F.Cu") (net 12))
 (segment (start 14.6868 3.7032) (end 14.6868 1.4482) (width 0.25) (layer "F.Cu") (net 12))
 (segment (start 14.6868 1.4482) (end 14.75 1.385) (width 0.25) (layer "F.Cu") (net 12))
 (segment (start 9.9125 6.4) (end 10.6375 7.125) (width 0.25) (layer "F.Cu") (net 15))
 (segment (start 10.6375 7.125) (end 12.15 7.125) (width 0.25) (layer "F.Cu") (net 15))
 (segment (start 14.2545 14.7788) (end 14.2545 16.2954) (width 0.25) (layer "F.Cu") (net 9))
 (segment (start 14.1 16.4499) (end 14.1 17.47) (width 0.25) (layer "F.Cu") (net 9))
 (segment (start 9.8875 10.8) (end 9.8875 10.9313) (width 0.25) (layer "F.Cu") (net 9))
 (segment (start 14.2545 16.2954) (end 14.1 16.4499) (width 0.25) (layer "F.Cu") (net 9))
 (segment (start 13.641 14.1653) (end 14.2545 14.7788) (width 0.25) (layer "F.Cu") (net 9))
 (segment (start 9.8875 10.9313) (end 13.1215 14.1653) (width 0.25) (layer "F.Cu") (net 9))
 (segment (start 13.1215 14.1653) (end 13.641 14.1653) (width 0.25) (layer "F.Cu") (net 9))
 (segment (start 14.75 10.6184) (end 12.7316 8.6) (width 0.25) (layer "F.Cu") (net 3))
 (segment (start 14.75 11.73) (end 14.75 10.6184) (width 0.25) (layer "F.Cu") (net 3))
 (segment (start 12.7316 8.6) (end 9.9125 8.6) (width 0.25) (layer "F.Cu") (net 3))
 (segment (start 12.15 15.2375) (end 9.9125 13) (width 0.25) (layer "F.Cu") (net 7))
 (segment (start 12.15 17.47) (end 12.15 15.2375) (width 0.25) (layer "F.Cu") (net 7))
 (segment (start 11.6233 9.7556) (end 12.8 10.9323) (width 0.25) (layer "F.Cu") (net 5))
 (segment (start 9.0312 10.0886) (end 9.3642 9.7556) (width 0.25) (layer "F.Cu") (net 5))
 (segment (start 9.3642 9.7556) (end 11.6233 9.7556) (width 0.25) (layer "F.Cu") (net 5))
 (segment (start 12.8 10.9323) (end 12.8 11.73) (width 0.25) (layer "F.Cu") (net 5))
 (segment (start 9.0312 14.3187) (end 9.0312 10.0886) (width 0.25) (layer "F.Cu") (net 5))
 (segment (start 9.9125 15.2) (end 9.0312 14.3187) (width 0.25) (layer "F.Cu") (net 5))
 (segment (start 5.1314 7.3286) (end 1.7 7.3286) (width 0.25) (layer "F.Cu") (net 14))
 (segment (start 11.06 5.51) (end 10.71 5.16) (width 0.25) (layer "F.Cu") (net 14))
 (segment (start 12.8 2.2318) (end 12.2542 2.7776) (width 0.25) (layer "F.Cu") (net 14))
 (segment (start 12.8 1.385) (end 12.8 2.2318) (width 0.25) (layer "F.Cu") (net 14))
 (segment (start 7.3 5.16) (end 5.1314 7.3286) (width 0.25) (layer "F.Cu") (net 14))
 (segment (start 10.71 5.16) (end 7.3 5.16) (width 0.25) (layer "F.Cu") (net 14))
 (segment (start 12.2542 2.7776) (end 12.1502 2.7776) (width 0.25) (layer "F.Cu") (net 14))
 (via (at 12.1502 2.7776) (size 0.8) (drill 0.4) (layers "F.Cu" "B.Cu") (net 14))
 (via (at 11.06 5.51) (size 0.8) (drill 0.4) (layers "F.Cu" "B.Cu") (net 14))
 (segment (start 11.06 5.51) (end 11.06 3.8678) (width 0.25) (layer "B.Cu") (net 14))
 (segment (start 11.06 3.8678) (end 12.1502 2.7776) (width 0.25) (layer "B.Cu") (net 14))
 (segment (start 1.91 3.51) (end 1.7 3.3) (width 0.25) (layer "F.Cu") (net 24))
 (segment (start 4.16 3.9) (end 3.56 3.3) (width 0.25) (layer "F.Cu") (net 24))
 (segment (start 3.56 3.3) (end 1.7 3.3) (width 0.25) (layer "F.Cu") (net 24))
 (segment (start 7.95 3.9) (end 4.16 3.9) (width 0.25) (layer "F.Cu") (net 24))
 (segment (start 17.9233 2.0767) (end 18.6 1.4) (width 0.25) (layer "F.Cu") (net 21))
 (segment (start 19.25 4.956) (end 17.9233 4.956) (width 0.25) (layer "F.Cu") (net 21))
 (segment (start 17.9233 4.956) (end 17.9233 2.0767) (width 0.25) (layer "F.Cu") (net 21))
 (segment (start 8.0875 6.4) (end 5.1446 9.3429) (width 0.25) (layer "F.Cu") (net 23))
 (segment (start 5.1446 9.3429) (end 1.7 9.3429) (width 0.25) (layer "F.Cu") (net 23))
 (segment (start 8.0875 8.6) (end 5.3304 11.3571) (width 0.25) (layer "F.Cu") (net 20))
 (segment (start 5.3304 11.3571) (end 1.7 11.3571) (width 0.25) (layer "F.Cu") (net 20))
 (segment (start 5.4911 13.3714) (end 1.7 13.3714) (width 0.25) (layer "F.Cu") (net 19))
 (segment (start 8.0625 10.8) (end 5.4911 13.3714) (width 0.25) (layer "F.Cu") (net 19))
 (segment (start 5.7018 15.3857) (end 1.7 15.3857) (width 0.25) (layer "F.Cu") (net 25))
 (segment (start 8.0875 13) (end 5.7018 15.3857) (width 0.25) (layer "F.Cu") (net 25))
 (segment (start 5.8875 17.4) (end 1.7 17.4) (width 0.25) (layer "F.Cu") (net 22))
 (segment (start 8.0875 15.2) (end 5.8875 17.4) (width 0.25) (layer "F.Cu") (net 22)))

